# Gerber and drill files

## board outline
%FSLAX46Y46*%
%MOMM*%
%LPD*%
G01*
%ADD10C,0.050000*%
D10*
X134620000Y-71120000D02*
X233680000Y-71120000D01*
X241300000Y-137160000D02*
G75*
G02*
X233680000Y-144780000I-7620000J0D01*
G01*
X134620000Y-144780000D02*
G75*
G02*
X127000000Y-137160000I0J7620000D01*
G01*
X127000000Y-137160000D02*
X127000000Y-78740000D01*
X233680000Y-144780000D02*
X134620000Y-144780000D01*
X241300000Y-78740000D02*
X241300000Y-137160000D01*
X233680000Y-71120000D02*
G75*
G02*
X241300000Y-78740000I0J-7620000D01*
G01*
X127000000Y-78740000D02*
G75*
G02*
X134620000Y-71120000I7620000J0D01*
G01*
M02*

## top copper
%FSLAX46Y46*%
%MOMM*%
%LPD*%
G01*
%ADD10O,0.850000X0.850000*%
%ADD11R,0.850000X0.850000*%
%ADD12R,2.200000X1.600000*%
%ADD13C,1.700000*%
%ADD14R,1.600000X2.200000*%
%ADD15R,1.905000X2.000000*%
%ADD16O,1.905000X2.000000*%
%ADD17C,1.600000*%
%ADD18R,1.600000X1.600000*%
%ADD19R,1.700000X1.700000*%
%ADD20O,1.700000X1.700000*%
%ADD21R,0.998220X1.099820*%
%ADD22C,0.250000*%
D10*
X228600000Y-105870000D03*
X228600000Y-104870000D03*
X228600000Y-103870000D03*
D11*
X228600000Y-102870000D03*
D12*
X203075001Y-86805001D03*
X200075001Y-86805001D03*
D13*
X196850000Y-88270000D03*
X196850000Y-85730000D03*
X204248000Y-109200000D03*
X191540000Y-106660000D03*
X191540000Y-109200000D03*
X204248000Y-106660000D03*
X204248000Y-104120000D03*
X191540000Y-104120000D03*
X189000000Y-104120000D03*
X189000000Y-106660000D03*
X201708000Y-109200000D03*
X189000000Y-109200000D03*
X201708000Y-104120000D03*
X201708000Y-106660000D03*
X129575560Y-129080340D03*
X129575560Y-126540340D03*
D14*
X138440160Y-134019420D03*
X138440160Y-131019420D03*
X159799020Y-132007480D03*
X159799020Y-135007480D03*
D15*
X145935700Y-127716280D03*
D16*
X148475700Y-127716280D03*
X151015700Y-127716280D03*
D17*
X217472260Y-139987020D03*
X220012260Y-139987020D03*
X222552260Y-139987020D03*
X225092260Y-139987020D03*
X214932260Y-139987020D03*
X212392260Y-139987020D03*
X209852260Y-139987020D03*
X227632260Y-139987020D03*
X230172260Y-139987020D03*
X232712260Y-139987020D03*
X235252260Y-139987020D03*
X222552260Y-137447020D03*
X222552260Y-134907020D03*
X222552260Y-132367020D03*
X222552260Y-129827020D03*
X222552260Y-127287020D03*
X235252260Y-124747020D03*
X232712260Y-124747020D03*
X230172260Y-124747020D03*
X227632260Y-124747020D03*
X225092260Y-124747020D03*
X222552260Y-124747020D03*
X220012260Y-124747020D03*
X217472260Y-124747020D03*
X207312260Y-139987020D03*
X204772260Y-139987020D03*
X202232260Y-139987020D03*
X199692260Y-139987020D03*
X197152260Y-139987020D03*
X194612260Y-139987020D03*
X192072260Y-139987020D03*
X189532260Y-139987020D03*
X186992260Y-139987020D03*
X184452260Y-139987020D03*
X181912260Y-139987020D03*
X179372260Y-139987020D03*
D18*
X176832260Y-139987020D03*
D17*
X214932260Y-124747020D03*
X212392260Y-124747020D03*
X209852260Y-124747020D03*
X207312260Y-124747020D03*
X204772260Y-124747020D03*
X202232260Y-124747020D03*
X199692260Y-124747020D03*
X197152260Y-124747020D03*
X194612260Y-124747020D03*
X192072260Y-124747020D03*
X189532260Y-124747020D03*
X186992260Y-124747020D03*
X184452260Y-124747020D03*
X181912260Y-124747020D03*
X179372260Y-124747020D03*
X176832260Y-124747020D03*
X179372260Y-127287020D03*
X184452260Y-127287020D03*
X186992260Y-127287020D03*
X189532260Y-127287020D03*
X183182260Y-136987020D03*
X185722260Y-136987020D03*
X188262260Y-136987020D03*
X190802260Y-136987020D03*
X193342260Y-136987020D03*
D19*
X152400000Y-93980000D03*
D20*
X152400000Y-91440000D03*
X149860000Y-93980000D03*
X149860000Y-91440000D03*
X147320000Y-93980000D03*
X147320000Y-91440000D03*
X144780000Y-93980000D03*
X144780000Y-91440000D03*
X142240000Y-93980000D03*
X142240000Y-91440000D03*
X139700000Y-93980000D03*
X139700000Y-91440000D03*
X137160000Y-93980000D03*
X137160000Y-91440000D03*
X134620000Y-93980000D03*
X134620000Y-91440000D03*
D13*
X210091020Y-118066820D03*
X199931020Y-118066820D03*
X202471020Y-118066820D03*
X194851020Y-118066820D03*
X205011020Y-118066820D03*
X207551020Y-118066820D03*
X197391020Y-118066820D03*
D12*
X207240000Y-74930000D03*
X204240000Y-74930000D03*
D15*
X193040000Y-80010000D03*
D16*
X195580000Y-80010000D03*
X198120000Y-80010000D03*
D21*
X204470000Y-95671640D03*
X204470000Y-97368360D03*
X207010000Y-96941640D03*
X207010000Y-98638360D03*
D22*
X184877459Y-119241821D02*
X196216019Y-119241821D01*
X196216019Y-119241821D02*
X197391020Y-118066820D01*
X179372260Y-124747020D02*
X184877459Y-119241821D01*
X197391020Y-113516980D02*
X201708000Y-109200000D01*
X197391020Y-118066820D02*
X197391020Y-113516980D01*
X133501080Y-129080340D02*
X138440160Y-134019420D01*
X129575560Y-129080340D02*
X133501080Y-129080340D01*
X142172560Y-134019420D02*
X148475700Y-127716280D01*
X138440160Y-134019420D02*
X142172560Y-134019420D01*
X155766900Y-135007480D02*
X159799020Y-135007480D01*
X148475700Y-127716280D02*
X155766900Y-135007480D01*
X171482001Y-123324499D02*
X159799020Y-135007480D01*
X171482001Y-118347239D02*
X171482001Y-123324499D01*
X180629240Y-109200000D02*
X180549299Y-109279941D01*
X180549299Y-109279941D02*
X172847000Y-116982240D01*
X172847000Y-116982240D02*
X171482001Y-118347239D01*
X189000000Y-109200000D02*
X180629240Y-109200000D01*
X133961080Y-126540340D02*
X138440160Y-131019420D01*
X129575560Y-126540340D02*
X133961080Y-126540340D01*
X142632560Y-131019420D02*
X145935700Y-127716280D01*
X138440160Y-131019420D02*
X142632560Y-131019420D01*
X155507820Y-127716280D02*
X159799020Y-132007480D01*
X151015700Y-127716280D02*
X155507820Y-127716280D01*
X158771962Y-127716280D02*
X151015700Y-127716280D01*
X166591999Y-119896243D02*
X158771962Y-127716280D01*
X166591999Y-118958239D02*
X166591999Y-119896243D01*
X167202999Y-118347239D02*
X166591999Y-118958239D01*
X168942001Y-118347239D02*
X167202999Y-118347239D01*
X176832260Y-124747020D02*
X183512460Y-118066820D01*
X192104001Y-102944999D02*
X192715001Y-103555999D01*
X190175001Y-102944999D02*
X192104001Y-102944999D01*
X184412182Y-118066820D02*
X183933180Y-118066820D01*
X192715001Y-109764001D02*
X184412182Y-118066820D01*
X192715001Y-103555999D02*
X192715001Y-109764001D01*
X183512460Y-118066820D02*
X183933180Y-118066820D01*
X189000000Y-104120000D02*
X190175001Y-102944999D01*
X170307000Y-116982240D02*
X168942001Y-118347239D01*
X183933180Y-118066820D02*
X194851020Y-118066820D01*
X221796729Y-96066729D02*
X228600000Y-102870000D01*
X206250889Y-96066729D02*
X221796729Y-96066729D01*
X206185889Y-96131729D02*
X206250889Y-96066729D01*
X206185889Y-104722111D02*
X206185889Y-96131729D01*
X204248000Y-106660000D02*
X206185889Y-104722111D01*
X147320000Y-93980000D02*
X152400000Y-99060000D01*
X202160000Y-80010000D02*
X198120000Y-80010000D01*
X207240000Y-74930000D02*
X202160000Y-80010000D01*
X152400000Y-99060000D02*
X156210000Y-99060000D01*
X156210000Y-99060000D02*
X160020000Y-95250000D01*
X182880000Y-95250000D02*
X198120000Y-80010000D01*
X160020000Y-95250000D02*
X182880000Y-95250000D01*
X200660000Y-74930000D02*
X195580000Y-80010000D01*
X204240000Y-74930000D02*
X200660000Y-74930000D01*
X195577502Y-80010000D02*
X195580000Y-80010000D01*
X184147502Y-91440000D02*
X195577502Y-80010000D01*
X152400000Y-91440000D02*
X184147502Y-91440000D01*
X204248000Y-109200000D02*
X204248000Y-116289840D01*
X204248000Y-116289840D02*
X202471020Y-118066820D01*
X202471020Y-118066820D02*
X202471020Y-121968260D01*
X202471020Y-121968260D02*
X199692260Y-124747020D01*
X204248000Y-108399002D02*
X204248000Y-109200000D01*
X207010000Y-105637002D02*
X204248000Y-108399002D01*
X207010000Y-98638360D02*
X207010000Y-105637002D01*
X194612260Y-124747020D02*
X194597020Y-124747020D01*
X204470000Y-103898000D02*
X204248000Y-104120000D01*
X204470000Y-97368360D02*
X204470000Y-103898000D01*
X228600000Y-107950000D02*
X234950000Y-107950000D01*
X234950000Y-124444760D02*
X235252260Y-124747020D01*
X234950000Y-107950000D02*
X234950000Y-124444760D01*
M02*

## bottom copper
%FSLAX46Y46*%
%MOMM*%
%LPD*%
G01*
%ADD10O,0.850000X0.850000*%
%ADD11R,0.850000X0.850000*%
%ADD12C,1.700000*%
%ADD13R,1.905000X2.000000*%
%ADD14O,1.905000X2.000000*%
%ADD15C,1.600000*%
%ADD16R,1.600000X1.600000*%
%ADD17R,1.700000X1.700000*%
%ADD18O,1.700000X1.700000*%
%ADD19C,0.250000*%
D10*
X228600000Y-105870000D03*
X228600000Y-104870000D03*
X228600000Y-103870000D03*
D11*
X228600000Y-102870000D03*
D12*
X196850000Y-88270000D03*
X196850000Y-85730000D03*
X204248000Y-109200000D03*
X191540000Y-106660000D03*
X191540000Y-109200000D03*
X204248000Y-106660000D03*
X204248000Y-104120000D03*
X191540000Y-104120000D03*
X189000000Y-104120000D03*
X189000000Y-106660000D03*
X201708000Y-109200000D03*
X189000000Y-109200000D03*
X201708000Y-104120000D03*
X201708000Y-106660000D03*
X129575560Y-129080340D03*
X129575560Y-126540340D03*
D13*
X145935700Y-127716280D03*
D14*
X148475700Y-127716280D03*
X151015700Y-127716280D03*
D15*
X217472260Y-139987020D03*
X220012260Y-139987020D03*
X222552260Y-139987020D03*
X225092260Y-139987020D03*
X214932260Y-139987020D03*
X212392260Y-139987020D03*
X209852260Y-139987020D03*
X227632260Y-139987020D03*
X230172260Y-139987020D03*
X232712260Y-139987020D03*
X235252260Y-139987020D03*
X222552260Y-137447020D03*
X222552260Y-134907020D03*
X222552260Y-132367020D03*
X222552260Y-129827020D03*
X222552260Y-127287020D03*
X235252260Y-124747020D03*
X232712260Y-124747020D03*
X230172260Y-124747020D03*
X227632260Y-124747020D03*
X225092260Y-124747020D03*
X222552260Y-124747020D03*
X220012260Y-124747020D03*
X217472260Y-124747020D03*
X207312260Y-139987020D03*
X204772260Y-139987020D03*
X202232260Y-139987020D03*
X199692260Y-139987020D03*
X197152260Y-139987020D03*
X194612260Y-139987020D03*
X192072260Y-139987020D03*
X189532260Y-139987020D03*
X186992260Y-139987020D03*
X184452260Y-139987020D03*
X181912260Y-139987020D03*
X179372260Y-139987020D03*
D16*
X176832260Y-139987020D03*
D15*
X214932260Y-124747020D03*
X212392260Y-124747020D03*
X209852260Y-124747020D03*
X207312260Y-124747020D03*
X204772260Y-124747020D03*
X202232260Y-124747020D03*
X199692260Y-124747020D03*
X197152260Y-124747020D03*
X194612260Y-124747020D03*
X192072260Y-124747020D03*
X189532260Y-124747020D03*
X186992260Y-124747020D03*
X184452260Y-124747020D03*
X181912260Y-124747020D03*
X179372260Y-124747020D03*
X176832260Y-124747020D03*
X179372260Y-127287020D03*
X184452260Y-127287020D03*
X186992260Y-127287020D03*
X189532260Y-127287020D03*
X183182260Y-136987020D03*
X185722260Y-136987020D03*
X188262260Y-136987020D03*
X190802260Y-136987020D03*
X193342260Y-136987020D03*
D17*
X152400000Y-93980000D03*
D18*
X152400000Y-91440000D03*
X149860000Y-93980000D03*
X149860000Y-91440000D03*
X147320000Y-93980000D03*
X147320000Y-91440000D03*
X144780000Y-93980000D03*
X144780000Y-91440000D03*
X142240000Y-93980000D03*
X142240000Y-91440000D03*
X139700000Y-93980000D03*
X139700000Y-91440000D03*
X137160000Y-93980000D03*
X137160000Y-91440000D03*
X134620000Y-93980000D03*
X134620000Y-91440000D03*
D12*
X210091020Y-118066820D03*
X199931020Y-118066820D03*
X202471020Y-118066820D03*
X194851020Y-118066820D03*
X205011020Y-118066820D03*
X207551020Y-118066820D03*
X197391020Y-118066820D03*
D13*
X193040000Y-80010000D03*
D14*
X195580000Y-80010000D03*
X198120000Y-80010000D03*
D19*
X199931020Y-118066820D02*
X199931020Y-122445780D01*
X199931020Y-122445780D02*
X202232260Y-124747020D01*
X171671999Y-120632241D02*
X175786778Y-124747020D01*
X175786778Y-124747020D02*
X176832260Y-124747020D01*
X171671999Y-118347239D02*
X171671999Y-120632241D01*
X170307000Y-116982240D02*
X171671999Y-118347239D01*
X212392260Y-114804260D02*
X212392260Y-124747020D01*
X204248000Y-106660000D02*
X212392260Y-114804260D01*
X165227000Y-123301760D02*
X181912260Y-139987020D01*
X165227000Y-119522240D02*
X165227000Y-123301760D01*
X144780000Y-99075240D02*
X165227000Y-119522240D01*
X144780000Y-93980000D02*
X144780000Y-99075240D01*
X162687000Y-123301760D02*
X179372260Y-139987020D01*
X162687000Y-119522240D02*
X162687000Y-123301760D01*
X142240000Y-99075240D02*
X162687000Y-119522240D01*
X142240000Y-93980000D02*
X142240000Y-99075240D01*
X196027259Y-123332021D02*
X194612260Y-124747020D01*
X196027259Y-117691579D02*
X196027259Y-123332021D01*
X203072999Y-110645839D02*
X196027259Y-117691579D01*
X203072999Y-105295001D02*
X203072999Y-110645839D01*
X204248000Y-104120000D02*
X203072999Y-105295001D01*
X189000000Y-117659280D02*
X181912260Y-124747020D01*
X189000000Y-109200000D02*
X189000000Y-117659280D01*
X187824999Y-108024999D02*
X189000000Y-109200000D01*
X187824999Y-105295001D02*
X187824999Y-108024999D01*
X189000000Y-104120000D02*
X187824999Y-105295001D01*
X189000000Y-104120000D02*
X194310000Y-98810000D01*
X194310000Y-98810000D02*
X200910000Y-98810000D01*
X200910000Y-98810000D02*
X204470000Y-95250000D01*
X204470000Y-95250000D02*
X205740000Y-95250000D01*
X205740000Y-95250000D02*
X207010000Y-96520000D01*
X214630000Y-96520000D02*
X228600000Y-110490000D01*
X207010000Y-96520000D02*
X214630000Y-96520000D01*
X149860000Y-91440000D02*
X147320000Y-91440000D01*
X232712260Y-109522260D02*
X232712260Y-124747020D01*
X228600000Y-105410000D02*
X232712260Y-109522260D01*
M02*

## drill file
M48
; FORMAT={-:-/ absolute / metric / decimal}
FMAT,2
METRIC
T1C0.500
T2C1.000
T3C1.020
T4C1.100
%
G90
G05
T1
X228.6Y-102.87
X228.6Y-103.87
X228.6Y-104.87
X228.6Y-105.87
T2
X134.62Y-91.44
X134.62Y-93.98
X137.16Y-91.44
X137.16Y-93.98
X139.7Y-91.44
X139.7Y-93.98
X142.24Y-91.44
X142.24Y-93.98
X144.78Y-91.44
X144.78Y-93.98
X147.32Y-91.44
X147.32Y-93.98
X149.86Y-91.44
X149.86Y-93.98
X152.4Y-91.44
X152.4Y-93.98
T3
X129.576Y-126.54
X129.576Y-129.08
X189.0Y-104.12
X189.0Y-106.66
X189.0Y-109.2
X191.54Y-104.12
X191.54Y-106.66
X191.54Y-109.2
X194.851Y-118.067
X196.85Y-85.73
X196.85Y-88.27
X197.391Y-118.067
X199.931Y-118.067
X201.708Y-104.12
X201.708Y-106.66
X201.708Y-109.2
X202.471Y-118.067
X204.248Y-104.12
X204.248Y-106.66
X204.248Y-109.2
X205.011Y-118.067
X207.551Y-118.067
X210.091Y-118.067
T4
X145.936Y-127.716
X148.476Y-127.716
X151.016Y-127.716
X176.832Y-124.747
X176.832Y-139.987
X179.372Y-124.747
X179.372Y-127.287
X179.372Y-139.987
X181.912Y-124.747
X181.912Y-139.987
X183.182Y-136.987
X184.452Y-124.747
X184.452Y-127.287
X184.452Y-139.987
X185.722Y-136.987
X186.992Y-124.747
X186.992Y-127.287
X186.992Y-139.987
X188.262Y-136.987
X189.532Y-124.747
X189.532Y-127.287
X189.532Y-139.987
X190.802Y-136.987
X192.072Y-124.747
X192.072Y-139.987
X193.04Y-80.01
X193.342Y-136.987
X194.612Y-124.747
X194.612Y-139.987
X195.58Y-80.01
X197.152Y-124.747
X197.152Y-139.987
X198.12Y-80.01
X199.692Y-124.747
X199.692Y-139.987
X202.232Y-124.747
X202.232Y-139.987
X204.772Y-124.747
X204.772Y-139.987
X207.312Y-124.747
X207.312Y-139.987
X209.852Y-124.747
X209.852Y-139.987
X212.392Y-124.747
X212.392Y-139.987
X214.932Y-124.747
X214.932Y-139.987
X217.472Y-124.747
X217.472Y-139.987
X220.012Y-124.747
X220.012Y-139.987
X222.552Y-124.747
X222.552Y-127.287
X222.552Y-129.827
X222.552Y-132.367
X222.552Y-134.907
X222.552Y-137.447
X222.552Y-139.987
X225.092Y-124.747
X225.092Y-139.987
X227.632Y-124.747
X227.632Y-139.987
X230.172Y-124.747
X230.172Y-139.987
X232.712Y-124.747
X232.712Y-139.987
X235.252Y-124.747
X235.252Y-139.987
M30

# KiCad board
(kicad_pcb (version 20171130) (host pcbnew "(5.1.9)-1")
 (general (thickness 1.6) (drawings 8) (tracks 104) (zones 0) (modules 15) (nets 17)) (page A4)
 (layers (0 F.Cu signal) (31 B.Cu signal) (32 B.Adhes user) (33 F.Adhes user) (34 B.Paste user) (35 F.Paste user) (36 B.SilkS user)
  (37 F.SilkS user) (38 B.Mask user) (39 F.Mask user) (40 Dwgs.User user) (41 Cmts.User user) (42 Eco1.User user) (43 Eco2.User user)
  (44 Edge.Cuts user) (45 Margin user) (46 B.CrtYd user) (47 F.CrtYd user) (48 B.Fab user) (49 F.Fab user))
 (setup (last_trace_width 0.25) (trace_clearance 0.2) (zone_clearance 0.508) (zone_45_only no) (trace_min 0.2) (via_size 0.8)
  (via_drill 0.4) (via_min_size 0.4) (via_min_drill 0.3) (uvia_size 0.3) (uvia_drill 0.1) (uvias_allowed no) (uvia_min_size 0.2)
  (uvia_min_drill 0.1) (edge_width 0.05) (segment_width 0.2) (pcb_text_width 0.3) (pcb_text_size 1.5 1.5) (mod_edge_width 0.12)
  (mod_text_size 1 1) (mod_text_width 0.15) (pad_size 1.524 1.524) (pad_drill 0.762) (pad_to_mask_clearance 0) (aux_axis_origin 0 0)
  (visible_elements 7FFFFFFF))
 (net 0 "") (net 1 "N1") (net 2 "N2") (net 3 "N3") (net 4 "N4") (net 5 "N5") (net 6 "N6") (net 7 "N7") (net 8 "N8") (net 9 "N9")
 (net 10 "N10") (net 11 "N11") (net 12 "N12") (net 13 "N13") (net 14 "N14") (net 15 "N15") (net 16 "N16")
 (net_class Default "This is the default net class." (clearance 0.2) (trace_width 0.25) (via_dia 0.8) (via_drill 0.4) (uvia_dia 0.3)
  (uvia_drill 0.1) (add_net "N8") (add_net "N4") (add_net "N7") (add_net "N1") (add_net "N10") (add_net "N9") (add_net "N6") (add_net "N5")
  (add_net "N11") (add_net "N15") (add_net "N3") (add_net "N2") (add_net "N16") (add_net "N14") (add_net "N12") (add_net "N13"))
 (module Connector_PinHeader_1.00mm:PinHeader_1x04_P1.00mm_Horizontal (layer F.Cu) (at 228.6 102.87)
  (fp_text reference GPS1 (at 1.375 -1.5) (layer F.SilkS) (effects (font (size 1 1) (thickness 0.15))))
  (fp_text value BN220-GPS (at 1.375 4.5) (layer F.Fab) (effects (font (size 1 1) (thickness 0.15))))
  (pad 4 thru_hole oval (at 0 3) (size 0.85 0.85) (drill 0.5) (layers *.Cu *.Mask) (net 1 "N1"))
  (pad 3 thru_hole oval (at 0 2) (size 0.85 0.85) (drill 0.5) (layers *.Cu *.Mask) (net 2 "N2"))
  (pad 2 thru_hole oval (at 0 1) (size 0.85 0.85) (drill 0.5) (layers *.Cu *.Mask) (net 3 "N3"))
  (pad 1 thru_hole rect (at 0 0) (size 0.85 0.85) (drill 0.5) (layers *.Cu *.Mask) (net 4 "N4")))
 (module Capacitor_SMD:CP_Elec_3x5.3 (layer F.Cu) (at 201.575001 86.805001)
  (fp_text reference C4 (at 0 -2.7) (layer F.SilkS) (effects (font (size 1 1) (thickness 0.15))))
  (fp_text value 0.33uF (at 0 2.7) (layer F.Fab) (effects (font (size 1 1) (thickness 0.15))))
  (pad 2 smd rect (at 1.5 0) (size 2.2 1.6) (layers F.Cu F.Paste F.Mask) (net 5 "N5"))
  (pad 1 smd rect (at -1.5 0) (size 2.2 1.6) (layers F.Cu F.Paste F.Mask) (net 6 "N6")))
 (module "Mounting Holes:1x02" (layer F.Cu) (at 196.85 91.44)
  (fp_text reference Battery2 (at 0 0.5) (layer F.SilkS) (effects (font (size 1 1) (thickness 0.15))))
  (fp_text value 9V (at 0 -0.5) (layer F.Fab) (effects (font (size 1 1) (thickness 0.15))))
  (pad 1 thru_hole circle (at 0 -3.17) (size 1.7 1.7) (drill 1.02) (layers *.Cu *.Mask) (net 6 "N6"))
  (pad 2 thru_hole circle (at 0 -5.71) (size 1.7 1.7) (drill 1.02) (layers *.Cu *.Mask) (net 5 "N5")))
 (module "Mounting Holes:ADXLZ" (layer F.Cu) (at 189 109.2)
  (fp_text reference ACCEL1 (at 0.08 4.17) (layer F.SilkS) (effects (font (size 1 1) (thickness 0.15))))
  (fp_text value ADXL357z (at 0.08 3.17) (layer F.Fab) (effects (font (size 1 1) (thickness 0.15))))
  (pad 3 thru_hole circle (at 15.248 0) (size 1.7 1.7) (drill 1.02) (layers *.Cu *.Mask) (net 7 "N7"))
  (pad 13 thru_hole circle (at 2.54 -2.54) (size 1.7 1.7) (drill 1.02) (layers *.Cu *.Mask))
  (pad 14 thru_hole circle (at 2.54 0) (size 1.7 1.7) (drill 1.02) (layers *.Cu *.Mask))
  (pad 2 thru_hole circle (at 15.248 -2.54) (size 1.7 1.7) (drill 1.02) (layers *.Cu *.Mask) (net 4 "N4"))
  (pad 1 thru_hole circle (at 15.248 -5.08) (size 1.7 1.7) (drill 1.02) (layers *.Cu *.Mask) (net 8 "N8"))
  (pad 12 thru_hole circle (at 2.54 -5.08) (size 1.7 1.7) (drill 1.02) (layers *.Cu *.Mask))
  (pad 5 thru_hole circle (at 0 -5.08) (size 1.7 1.7) (drill 1.02) (layers *.Cu *.Mask) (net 1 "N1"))
  (pad 11 thru_hole circle (at 0 -2.54) (size 1.7 1.7) (drill 1.02) (layers *.Cu *.Mask))
  (pad 4 thru_hole circle (at 12.708 0) (size 1.7 1.7) (drill 1.02) (layers *.Cu *.Mask))
  (pad 6 thru_hole circle (at 0 0) (size 1.7 1.7) (drill 1.02) (layers *.Cu *.Mask) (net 1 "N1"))
  (pad 10 thru_hole circle (at 12.708 -5.08) (size 1.7 1.7) (drill 1.02) (layers *.Cu *.Mask))
  (pad 8 thru_hole circle (at 12.708 -2.54) (size 1.7 1.7) (drill 1.02) (layers *.Cu *.Mask)))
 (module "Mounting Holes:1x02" (layer F.Cu) (at 129.57556 123.37034 180)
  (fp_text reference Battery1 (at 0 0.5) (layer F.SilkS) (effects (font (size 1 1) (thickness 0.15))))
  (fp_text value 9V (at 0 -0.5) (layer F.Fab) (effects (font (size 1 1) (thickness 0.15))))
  (pad 2 thru_hole circle (at 0 -5.71 180) (size 1.7 1.7) (drill 1.02) (layers *.Cu *.Mask) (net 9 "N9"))
  (pad 1 thru_hole circle (at 0 -3.17 180) (size 1.7 1.7) (drill 1.02) (layers *.Cu *.Mask) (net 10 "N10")))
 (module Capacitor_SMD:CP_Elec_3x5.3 (layer F.Cu) (at 138.44016 132.51942 270)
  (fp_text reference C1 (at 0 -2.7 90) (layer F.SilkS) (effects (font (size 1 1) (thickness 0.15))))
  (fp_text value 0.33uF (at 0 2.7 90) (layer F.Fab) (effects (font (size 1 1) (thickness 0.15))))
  (pad 2 smd rect (at 1.5 0 270) (size 2.2 1.6) (layers F.Cu F.Paste F.Mask) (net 9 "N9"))
  (pad 1 smd rect (at -1.5 0 270) (size 2.2 1.6) (layers F.Cu F.Paste F.Mask) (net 10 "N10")))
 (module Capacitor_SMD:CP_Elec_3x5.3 (layer F.Cu) (at 159.79902 133.50748 270)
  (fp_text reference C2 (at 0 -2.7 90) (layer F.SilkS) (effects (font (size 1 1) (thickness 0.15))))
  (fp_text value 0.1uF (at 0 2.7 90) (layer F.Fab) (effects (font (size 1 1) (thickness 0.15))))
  (pad 1 smd rect (at -1.5 0 270) (size 2.2 1.6) (layers F.Cu F.Paste F.Mask) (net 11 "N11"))
  (pad 2 smd rect (at 1.5 0 270) (size 2.2 1.6) (layers F.Cu F.Paste F.Mask) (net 9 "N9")))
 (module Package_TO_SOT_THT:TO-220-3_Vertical (layer F.Cu) (at 145.9357 127.71628)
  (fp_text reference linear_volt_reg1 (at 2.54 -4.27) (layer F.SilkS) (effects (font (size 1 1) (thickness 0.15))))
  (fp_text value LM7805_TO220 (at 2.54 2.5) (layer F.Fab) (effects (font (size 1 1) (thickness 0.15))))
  (pad 1 thru_hole rect (at 0 0) (size 1.905 2) (drill 1.1) (layers *.Cu *.Mask) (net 10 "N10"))
  (pad 2 thru_hole oval (at 2.54 0) (size 1.905 2) (drill 1.1) (layers *.Cu *.Mask) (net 9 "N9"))
  (pad 3 thru_hole oval (at 5.08 0) (size 1.905 2) (drill 1.1) (layers *.Cu *.Mask) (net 11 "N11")))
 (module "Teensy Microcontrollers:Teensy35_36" (layer F.Cu) (at 206.04226 132.36702)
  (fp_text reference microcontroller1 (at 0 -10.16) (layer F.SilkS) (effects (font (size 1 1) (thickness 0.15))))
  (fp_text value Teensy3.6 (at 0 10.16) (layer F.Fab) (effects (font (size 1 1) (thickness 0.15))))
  (pad 17 thru_hole circle (at 11.43 7.62) (size 1.6 1.6) (drill 1.1) (layers *.Cu *.Mask))
  (pad 18 thru_hole circle (at 13.97 7.62) (size 1.6 1.6) (drill 1.1) (layers *.Cu *.Mask))
  (pad 19 thru_hole circle (at 16.51 7.62) (size 1.6 1.6) (drill 1.1) (layers *.Cu *.Mask))
  (pad 20 thru_hole circle (at 19.05 7.62) (size 1.6 1.6) (drill 1.1) (layers *.Cu *.Mask))
  (pad 16 thru_hole circle (at 8.89 7.62) (size 1.6 1.6) (drill 1.1) (layers *.Cu *.Mask))
  (pad 15 thru_hole circle (at 6.35 7.62) (size 1.6 1.6) (drill 1.1) (layers *.Cu *.Mask))
  (pad 14 thru_hole circle (at 3.81 7.62) (size 1.6 1.6) (drill 1.1) (layers *.Cu *.Mask))
  (pad 21 thru_hole circle (at 21.59 7.62) (size 1.6 1.6) (drill 1.1) (layers *.Cu *.Mask))
  (pad 22 thru_hole circle (at 24.13 7.62) (size 1.6 1.6) (drill 1.1) (layers *.Cu *.Mask))
  (pad 23 thru_hole circle (at 26.67 7.62) (size 1.6 1.6) (drill 1.1) (layers *.Cu *.Mask))
  (pad 24 thru_hole circle (at 29.21 7.62) (size 1.6 1.6) (drill 1.1) (layers *.Cu *.Mask))
  (pad 25 thru_hole circle (at 16.51 5.08) (size 1.6 1.6) (drill 1.1) (layers *.Cu *.Mask))
  (pad 26 thru_hole circle (at 16.51 2.54) (size 1.6 1.6) (drill 1.1) (layers *.Cu *.Mask))
  (pad 27 thru_hole circle (at 16.51 0) (size 1.6 1.6) (drill 1.1) (layers *.Cu *.Mask))
  (pad 28 thru_hole circle (at 16.51 -2.54) (size 1.6 1.6) (drill 1.1) (layers *.Cu *.Mask))
  (pad 29 thru_hole circle (at 16.51 -5.08) (size 1.6 1.6) (drill 1.1) (layers *.Cu *.Mask))
  (pad 30 thru_hole circle (at 29.21 -7.62) (size 1.6 1.6) (drill 1.1) (layers *.Cu *.Mask) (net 2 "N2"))
  (pad 31 thru_hole circle (at 26.67 -7.62) (size 1.6 1.6) (drill 1.1) (layers *.Cu *.Mask) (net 3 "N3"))
  (pad 32 thru_hole circle (at 24.13 -7.62) (size 1.6 1.6) (drill 1.1) (layers *.Cu *.Mask))
  (pad 33 thru_hole circle (at 21.59 -7.62) (size 1.6 1.6) (drill 1.1) (layers *.Cu *.Mask))
  (pad 34 thru_hole circle (at 19.05 -7.62) (size 1.6 1.6) (drill 1.1) (layers *.Cu *.Mask))
  (pad 35 thru_hole circle (at 16.51 -7.62) (size 1.6 1.6) (drill 1.1) (layers *.Cu *.Mask))
  (pad 36 thru_hole circle (at 13.97 -7.62) (size 1.6 1.6) (drill 1.1) (layers *.Cu *.Mask))
  (pad 37 thru_hole circle (at 11.43 -7.62) (size 1.6 1.6) (drill 1.1) (layers *.Cu *.Mask))
  (pad 13 thru_hole circle (at 1.27 7.62) (size 1.6 1.6) (drill 1.1) (layers *.Cu *.Mask))
  (pad 12 thru_hole circle (at -1.27 7.62) (size 1.6 1.6) (drill 1.1) (layers *.Cu *.Mask))
  (pad 11 thru_hole circle (at -3.81 7.62) (size 1.6 1.6) (drill 1.1) (layers *.Cu *.Mask))
  (pad 10 thru_hole circle (at -6.35 7.62) (size 1.6 1.6) (drill 1.1) (layers *.Cu *.Mask))
  (pad 9 thru_hole circle (at -8.89 7.62) (size 1.6 1.6) (drill 1.1) (layers *.Cu *.Mask))
  (pad 8 thru_hole circle (at -11.43 7.62) (size 1.6 1.6) (drill 1.1) (layers *.Cu *.Mask))
  (pad 7 thru_hole circle (at -13.97 7.62) (size 1.6 1.6) (drill 1.1) (layers *.Cu *.Mask))
  (pad 6 thru_hole circle (at -16.51 7.62) (size 1.6 1.6) (drill 1.1) (layers *.Cu *.Mask))
  (pad 5 thru_hole circle (at -19.05 7.62) (size 1.6 1.6) (drill 1.1) (layers *.Cu *.Mask))
  (pad 4 thru_hole circle (at -21.59 7.62) (size 1.6 1.6) (drill 1.1) (layers *.Cu *.Mask))
  (pad 3 thru_hole circle (at -24.13 7.62) (size 1.6 1.6) (drill 1.1) (layers *.Cu *.Mask) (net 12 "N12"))
  (pad 2 thru_hole circle (at -26.67 7.62) (size 1.6 1.6) (drill 1.1) (layers *.Cu *.Mask) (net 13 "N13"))
  (pad 1 thru_hole rect (at -29.21 7.62) (size 1.6 1.6) (drill 1.1) (layers *.Cu *.Mask))
  (pad 38 thru_hole circle (at 8.89 -7.62) (size 1.6 1.6) (drill 1.1) (layers *.Cu *.Mask))
  (pad 39 thru_hole circle (at 6.35 -7.62) (size 1.6 1.6) (drill 1.1) (layers *.Cu *.Mask) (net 4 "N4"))
  (pad 40 thru_hole circle (at 3.81 -7.62) (size 1.6 1.6) (drill 1.1) (layers *.Cu *.Mask))
  (pad 41 thru_hole circle (at 1.27 -7.62) (size 1.6 1.6) (drill 1.1) (layers *.Cu *.Mask))
  (pad 42 thru_hole circle (at -1.27 -7.62) (size 1.6 1.6) (drill 1.1) (layers *.Cu *.Mask))
  (pad 43 thru_hole circle (at -3.81 -7.62) (size 1.6 1.6) (drill 1.1) (layers *.Cu *.Mask))
  (pad 44 thru_hole circle (at -6.35 -7.62) (size 1.6 1.6) (drill 1.1) (layers *.Cu *.Mask))
  (pad 45 thru_hole circle (at -8.89 -7.62) (size 1.6 1.6) (drill 1.1) (layers *.Cu *.Mask) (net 7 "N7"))
  (pad 46 thru_hole circle (at -11.43 -7.62) (size 1.6 1.6) (drill 1.1) (layers *.Cu *.Mask) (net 8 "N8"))
  (pad 47 thru_hole circle (at -13.97 -7.62) (size 1.6 1.6) (drill 1.1) (layers *.Cu *.Mask))
  (pad 48 thru_hole circle (at -16.51 -7.62) (size 1.6 1.6) (drill 1.1) (layers *.Cu *.Mask))
  (pad 49 thru_hole circle (at -19.05 -7.62) (size 1.6 1.6) (drill 1.1) (layers *.Cu *.Mask))
  (pad 50 thru_hole circle (at -21.59 -7.62) (size 1.6 1.6) (drill 1.1) (layers *.Cu *.Mask))
  (pad 51 thru_hole circle (at -24.13 -7.62) (size 1.6 1.6) (drill 1.1) (layers *.Cu *.Mask) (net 1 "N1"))
  (pad 52 thru_hole circle (at -26.67 -7.62) (size 1.6 1.6) (drill 1.1) (layers *.Cu *.Mask))
  (pad 53 thru_hole circle (at -29.21 -7.62) (size 1.6 1.6) (drill 1.1) (layers *.Cu *.Mask) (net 11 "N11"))
  (pad 54 thru_hole circle (at -26.67 -5.08) (size 1.6 1.6) (drill 1.1) (layers *.Cu *.Mask))
  (pad 55 thru_hole circle (at -21.59 -5.08) (size 1.6 1.6) (drill 1.1) (layers *.Cu *.Mask))
  (pad 56 thru_hole circle (at -19.05 -5.08) (size 1.6 1.6) (drill 1.1) (layers *.Cu *.Mask))
  (pad 57 thru_hole circle (at -16.51 -5.08) (size 1.6 1.6) (drill 1.1) (layers *.Cu *.Mask))
  (pad 58 thru_hole circle (at -22.86 4.62) (size 1.6 1.6) (drill 1.1) (layers *.Cu *.Mask))
  (pad 59 thru_hole circle (at -20.32 4.62) (size 1.6 1.6) (drill 1.1) (layers *.Cu *.Mask))
  (pad 60 thru_hole circle (at -17.78 4.62) (size 1.6 1.6) (drill 1.1) (layers *.Cu *.Mask))
  (pad 61 thru_hole circle (at -15.24 4.62) (size 1.6 1.6) (drill 1.1) (layers *.Cu *.Mask))
  (pad 62 thru_hole circle (at -12.7 4.62) (size 1.6 1.6) (drill 1.1) (layers *.Cu *.Mask)))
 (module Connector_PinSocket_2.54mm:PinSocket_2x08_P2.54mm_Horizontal (layer F.Cu) (at 152.4 93.98 270)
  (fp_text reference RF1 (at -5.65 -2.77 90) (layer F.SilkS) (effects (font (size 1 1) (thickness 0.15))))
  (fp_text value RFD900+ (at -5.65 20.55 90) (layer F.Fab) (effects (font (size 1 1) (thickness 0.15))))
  (pad 1 thru_hole rect (at 0 0 270) (size 1.7 1.7) (drill 1) (layers *.Cu *.Mask))
  (pad 2 thru_hole oval (at -2.54 0 270) (size 1.7 1.7) (drill 1) (layers *.Cu *.Mask) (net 5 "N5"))
  (pad 3 thru_hole oval (at 0 2.54 270) (size 1.7 1.7) (drill 1) (layers *.Cu *.Mask))
  (pad 4 thru_hole oval (at -2.54 2.54 270) (size 1.7 1.7) (drill 1) (layers *.Cu *.Mask) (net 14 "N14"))
  (pad 5 thru_hole oval (at 0 5.08 270) (size 1.7 1.7) (drill 1) (layers *.Cu *.Mask) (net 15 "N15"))
  (pad 6 thru_hole oval (at -2.54 5.08 270) (size 1.7 1.7) (drill 1) (layers *.Cu *.Mask) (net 14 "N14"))
  (pad 7 thru_hole oval (at 0 7.62 270) (size 1.7 1.7) (drill 1) (layers *.Cu *.Mask) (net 12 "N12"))
  (pad 8 thru_hole oval (at -2.54 7.62 270) (size 1.7 1.7) (drill 1) (layers *.Cu *.Mask))
  (pad 9 thru_hole oval (at 0 10.16 270) (size 1.7 1.7) (drill 1) (layers *.Cu *.Mask) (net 13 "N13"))
  (pad 10 thru_hole oval (at -2.54 10.16 270) (size 1.7 1.7) (drill 1) (layers *.Cu *.Mask))
  (pad 11 thru_hole oval (at 0 12.7 270) (size 1.7 1.7) (drill 1) (layers *.Cu *.Mask))
  (pad 12 thru_hole oval (at -2.54 12.7 270) (size 1.7 1.7) (drill 1) (layers *.Cu *.Mask))
  (pad 13 thru_hole oval (at 0 15.24 270) (size 1.7 1.7) (drill 1) (layers *.Cu *.Mask))
  (pad 14 thru_hole oval (at -2.54 15.24 270) (size 1.7 1.7) (drill 1) (layers *.Cu *.Mask))
  (pad 15 thru_hole oval (at 0 17.78 270) (size 1.7 1.7) (drill 1) (layers *.Cu *.Mask))
  (pad 16 thru_hole oval (at -2.54 17.78 270) (size 1.7 1.7) (drill 1) (layers *.Cu *.Mask)))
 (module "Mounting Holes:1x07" (layer F.Cu) (at 192.53102 118.08682 270)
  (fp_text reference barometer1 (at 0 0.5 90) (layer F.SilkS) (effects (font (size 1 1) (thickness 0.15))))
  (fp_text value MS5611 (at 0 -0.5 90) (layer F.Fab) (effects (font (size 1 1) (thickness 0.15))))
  (pad 7 thru_hole circle (at -0.02 -17.56 270) (size 1.7 1.7) (drill 1.02) (layers *.Cu *.Mask))
  (pad 3 thru_hole circle (at -0.02 -7.4 270) (size 1.7 1.7) (drill 1.02) (layers *.Cu *.Mask))
  (pad 4 thru_hole circle (at -0.02 -9.94 270) (size 1.7 1.7) (drill 1.02) (layers *.Cu *.Mask))
  (pad 1 thru_hole circle (at -0.02 -2.32 270) (size 1.7 1.7) (drill 1.02) (layers *.Cu *.Mask))
  (pad 5 thru_hole circle (at -0.02 -12.48 270) (size 1.7 1.7) (drill 1.02) (layers *.Cu *.Mask))
  (pad 6 thru_hole circle (at -0.02 -15.02 270) (size 1.7 1.7) (drill 1.02) (layers *.Cu *.Mask))
  (pad 2 thru_hole circle (at -0.02 -4.86 270) (size 1.7 1.7) (drill 1.02) (layers *.Cu *.Mask)))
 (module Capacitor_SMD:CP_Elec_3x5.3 (layer F.Cu) (at 205.74 74.93 180)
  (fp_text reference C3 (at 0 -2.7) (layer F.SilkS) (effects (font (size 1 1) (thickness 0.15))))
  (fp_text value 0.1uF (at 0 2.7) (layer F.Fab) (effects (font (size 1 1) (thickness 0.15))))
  (pad 1 smd rect (at -1.5 0 180) (size 2.2 1.6) (layers F.Cu F.Paste F.Mask) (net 15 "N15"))
  (pad 2 smd rect (at 1.5 0 180) (size 2.2 1.6) (layers F.Cu F.Paste F.Mask) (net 5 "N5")))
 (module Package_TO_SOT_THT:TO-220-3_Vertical (layer F.Cu) (at 193.04 80.01)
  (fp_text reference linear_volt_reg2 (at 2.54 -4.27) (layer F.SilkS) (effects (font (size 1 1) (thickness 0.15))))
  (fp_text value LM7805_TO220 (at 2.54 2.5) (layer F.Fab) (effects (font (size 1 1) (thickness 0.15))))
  (pad 1 thru_hole rect (at 0 0) (size 1.905 2) (drill 1.1) (layers *.Cu *.Mask) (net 6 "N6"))
  (pad 2 thru_hole oval (at 2.54 0) (size 1.905 2) (drill 1.1) (layers *.Cu *.Mask) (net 5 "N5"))
  (pad 3 thru_hole oval (at 5.08 0) (size 1.905 2) (drill 1.1) (layers *.Cu *.Mask) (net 15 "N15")))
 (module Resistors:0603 (layer F.Cu) (at 204.47 96.52 270)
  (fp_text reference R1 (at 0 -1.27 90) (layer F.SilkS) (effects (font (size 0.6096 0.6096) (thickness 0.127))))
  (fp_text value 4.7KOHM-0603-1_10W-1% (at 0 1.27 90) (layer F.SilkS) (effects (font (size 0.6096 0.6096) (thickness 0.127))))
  (pad 1 smd rect (at -0.84836 0 270) (size 1.09982 0.99822) (layers F.Cu F.Paste F.Mask) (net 1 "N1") (solder_mask_margin 0.1016))
  (pad 2 smd rect (at 0.84836 0 270) (size 1.09982 0.99822) (layers F.Cu F.Paste F.Mask) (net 8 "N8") (solder_mask_margin 0.1016)))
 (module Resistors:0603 (layer F.Cu) (at 207.01 97.79 90)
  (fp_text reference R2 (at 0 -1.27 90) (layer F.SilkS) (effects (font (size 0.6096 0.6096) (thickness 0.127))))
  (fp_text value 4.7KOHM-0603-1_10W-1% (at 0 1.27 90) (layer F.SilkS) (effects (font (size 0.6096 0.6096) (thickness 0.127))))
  (pad 2 smd rect (at 0.84836 0 90) (size 1.09982 0.99822) (layers F.Cu F.Paste F.Mask) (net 1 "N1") (solder_mask_margin 0.1016))
  (pad 1 smd rect (at -0.84836 0 90) (size 1.09982 0.99822) (layers F.Cu F.Paste F.Mask) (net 7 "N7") (solder_mask_margin 0.1016)))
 (gr_line (start 134.62 71.12) (end 233.68 71.12) (layer Edge.Cuts) (width 0.05))
 (gr_arc (start 233.68 137.16) (end 233.68 144.78) (angle -90) (layer Edge.Cuts) (width 0.05))
 (gr_arc (start 134.62 137.16) (end 127 137.16) (angle -90) (layer Edge.Cuts) (width 0.05))
 (gr_line (start 127 137.16) (end 127 78.74) (layer Edge.Cuts) (width 0.05))
 (gr_line (start 233.68 144.78) (end 134.62 144.78) (layer Edge.Cuts) (width 0.05))
 (gr_line (start 241.3 78.74) (end 241.3 137.16) (layer Edge.Cuts) (width 0.05))
 (gr_arc (start 233.68 78.74) (end 241.3 78.74) (angle -90) (layer Edge.Cuts) (width 0.05))
 (gr_arc (start 134.62 78.74) (end 134.62 71.12) (angle -90) (layer Edge.Cuts) (width 0.05))
 (segment (start 184.877459 119.241821) (end 196.216019 119.241821) (width 0.25) (layer F.Cu) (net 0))
 (segment (start 196.216019 119.241821) (end 197.39102 118.06682) (width 0.25) (layer F.Cu) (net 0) (status 20))
 (segment (start 179.37226 124.74702) (end 184.877459 119.241821) (width 0.25) (layer F.Cu) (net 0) (status 10))
 (segment (start 197.39102 113.51698) (end 201.708 109.2) (width 0.25) (layer F.Cu) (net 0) (status 20))
 (segment (start 197.39102 118.06682) (end 197.39102 113.51698) (width 0.25) (layer F.Cu) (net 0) (status 10))
 (segment (start 199.93102 118.06682) (end 199.93102 122.44578) (width 0.25) (layer B.Cu) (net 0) (status 10))
 (segment (start 199.93102 122.44578) (end 202.23226 124.74702) (width 0.25) (layer B.Cu) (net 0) (status 20))
 (segment (start 133.50108 129.08034) (end 138.44016 134.01942) (width 0.25) (layer F.Cu) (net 9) (status 20))
 (segment (start 129.57556 129.08034) (end 133.50108 129.08034) (width 0.25) (layer F.Cu) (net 9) (status 10))
 (segment (start 142.17256 134.01942) (end 148.4757 127.71628) (width 0.25) (layer F.Cu) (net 9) (status 20))
 (segment (start 138.44016 134.01942) (end 142.17256 134.01942) (width 0.25) (layer F.Cu) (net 9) (status 10))
 (segment (start 155.7669 135.00748) (end 159.79902 135.00748) (width 0.25) (layer F.Cu) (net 9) (status 20))
 (segment (start 148.4757 127.71628) (end 155.7669 135.00748) (width 0.25) (layer F.Cu) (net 9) (status 10))
 (segment (start 171.482001 123.324499) (end 159.79902 135.00748) (width 0.25) (layer F.Cu) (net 9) (status 20))
 (segment (start 171.482001 118.347239) (end 171.482001 123.324499) (width 0.25) (layer F.Cu) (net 9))
 (segment (start 180.62924 109.2) (end 180.549299 109.279941) (width 0.25) (layer F.Cu) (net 9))
 (segment (start 180.549299 109.279941) (end 172.847 116.98224) (width 0.25) (layer F.Cu) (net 9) (status 20))
 (segment (start 172.847 116.98224) (end 171.482001 118.347239) (width 0.25) (layer F.Cu) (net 9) (status 10))
 (segment (start 189 109.2) (end 180.62924 109.2) (width 0.25) (layer F.Cu) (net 9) (status 10))
 (segment (start 133.96108 126.54034) (end 138.44016 131.01942) (width 0.25) (layer F.Cu) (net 10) (status 20))
 (segment (start 129.57556 126.54034) (end 133.96108 126.54034) (width 0.25) (layer F.Cu) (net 10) (status 10))
 (segment (start 142.63256 131.01942) (end 145.9357 127.71628) (width 0.25) (layer F.Cu) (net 10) (status 20))
 (segment (start 138.44016 131.01942) (end 142.63256 131.01942) (width 0.25) (layer F.Cu) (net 10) (status 10))
 (segment (start 155.50782 127.71628) (end 159.79902 132.00748) (width 0.25) (layer F.Cu) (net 11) (status 20))
 (segment (start 151.0157 127.71628) (end 155.50782 127.71628) (width 0.25) (layer F.Cu) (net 11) (status 10))
 (segment (start 158.771962 127.71628) (end 151.0157 127.71628) (width 0.25) (layer F.Cu) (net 11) (status 20))
 (segment (start 166.591999 119.896243) (end 158.771962 127.71628) (width 0.25) (layer F.Cu) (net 11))
 (segment (start 166.591999 118.958239) (end 166.591999 119.896243) (width 0.25) (layer F.Cu) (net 11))
 (segment (start 167.202999 118.347239) (end 166.591999 118.958239) (width 0.25) (layer F.Cu) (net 11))
 (segment (start 168.942001 118.347239) (end 167.202999 118.347239) (width 0.25) (layer F.Cu) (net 11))
 (segment (start 171.671999 120.632241) (end 175.786778 124.74702) (width 0.25) (layer B.Cu) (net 11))
 (segment (start 175.786778 124.74702) (end 176.83226 124.74702) (width 0.25) (layer B.Cu) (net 11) (status 20))
 (segment (start 171.671999 118.347239) (end 171.671999 120.632241) (width 0.25) (layer B.Cu) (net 11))
 (segment (start 176.83226 124.74702) (end 183.51246 118.06682) (width 0.25) (layer F.Cu) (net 11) (status 10))
 (segment (start 192.104001 102.944999) (end 192.715001 103.555999) (width 0.25) (layer F.Cu) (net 11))
 (segment (start 190.175001 102.944999) (end 192.104001 102.944999) (width 0.25) (layer F.Cu) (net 11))
 (segment (start 184.412182 118.06682) (end 183.93318 118.06682) (width 0.25) (layer F.Cu) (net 11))
 (segment (start 192.715001 109.764001) (end 184.412182 118.06682) (width 0.25) (layer F.Cu) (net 11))
 (segment (start 192.715001 103.555999) (end 192.715001 109.764001) (width 0.25) (layer F.Cu) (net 11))
 (segment (start 183.51246 118.06682) (end 183.93318 118.06682) (width 0.25) (layer F.Cu) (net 11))
 (segment (start 189 104.12) (end 190.175001 102.944999) (width 0.25) (layer F.Cu) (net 11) (status 10))
 (segment (start 170.307 116.98224) (end 168.942001 118.347239) (width 0.25) (layer F.Cu) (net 11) (status 10))
 (segment (start 183.93318 118.06682) (end 194.85102 118.06682) (width 0.25) (layer F.Cu) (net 11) (status 20))
 (segment (start 170.307 116.98224) (end 171.671999 118.347239) (width 0.25) (layer B.Cu) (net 11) (status 10))
 (segment (start 221.796729 96.066729) (end 228.6 102.87) (width 0.25) (layer F.Cu) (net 4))
 (segment (start 206.250889 96.066729) (end 221.796729 96.066729) (width 0.25) (layer F.Cu) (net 4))
 (segment (start 206.185889 96.131729) (end 206.250889 96.066729) (width 0.25) (layer F.Cu) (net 4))
 (segment (start 206.185889 104.722111) (end 206.185889 96.131729) (width 0.25) (layer F.Cu) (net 4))
 (segment (start 204.248 106.66) (end 206.185889 104.722111) (width 0.25) (layer F.Cu) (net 4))
 (segment (start 212.39226 114.80426) (end 212.39226 124.74702) (width 0.25) (layer B.Cu) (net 4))
 (segment (start 204.248 106.66) (end 212.39226 114.80426) (width 0.25) (layer B.Cu) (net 4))
 (segment (start 165.227 123.30176) (end 181.91226 139.98702) (width 0.25) (layer B.Cu) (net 12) (status 20))
 (segment (start 165.227 119.52224) (end 165.227 123.30176) (width 0.25) (layer B.Cu) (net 12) (status 10))
 (segment (start 144.78 99.07524) (end 165.227 119.52224) (width 0.25) (layer B.Cu) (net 12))
 (segment (start 144.78 93.98) (end 144.78 99.07524) (width 0.25) (layer B.Cu) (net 12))
 (segment (start 162.687 123.30176) (end 179.37226 139.98702) (width 0.25) (layer B.Cu) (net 13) (status 20))
 (segment (start 162.687 119.52224) (end 162.687 123.30176) (width 0.25) (layer B.Cu) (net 13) (status 10))
 (segment (start 142.24 99.07524) (end 162.687 119.52224) (width 0.25) (layer B.Cu) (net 13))
 (segment (start 142.24 93.98) (end 142.24 99.07524) (width 0.25) (layer B.Cu) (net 13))
 (segment (start 147.32 93.98) (end 152.4 99.06) (width 0.25) (layer F.Cu) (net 15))
 (segment (start 202.16 80.01) (end 198.12 80.01) (width 0.25) (layer F.Cu) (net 15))
 (segment (start 207.24 74.93) (end 202.16 80.01) (width 0.25) (layer F.Cu) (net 15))
 (segment (start 152.4 99.06) (end 156.21 99.06) (width 0.25) (layer F.Cu) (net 15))
 (segment (start 156.21 99.06) (end 160.02 95.25) (width 0.25) (layer F.Cu) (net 15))
 (segment (start 182.88 95.25) (end 198.12 80.01) (width 0.25) (layer F.Cu) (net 15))
 (segment (start 160.02 95.25) (end 182.88 95.25) (width 0.25) (layer F.Cu) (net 15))
 (segment (start 200.66 74.93) (end 195.58 80.01) (width 0.25) (layer F.Cu) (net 5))
 (segment (start 204.24 74.93) (end 200.66 74.93) (width 0.25) (layer F.Cu) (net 5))
 (segment (start 195.577502 80.01) (end 195.58 80.01) (width 0.25) (layer F.Cu) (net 5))
 (segment (start 184.147502 91.44) (end 195.577502 80.01) (width 0.25) (layer F.Cu) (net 5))
 (segment (start 152.4 91.44) (end 184.147502 91.44) (width 0.25) (layer F.Cu) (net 5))
 (segment (start 204.248 109.2) (end 204.248 116.28984) (width 0.25) (layer F.Cu) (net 7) (status 10))
 (segment (start 204.248 116.28984) (end 202.47102 118.06682) (width 0.25) (layer F.Cu) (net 7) (status 20))
 (segment (start 202.47102 118.06682) (end 202.47102 121.96826) (width 0.25) (layer F.Cu) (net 7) (status 10))
 (segment (start 202.47102 121.96826) (end 199.69226 124.74702) (width 0.25) (layer F.Cu) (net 7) (status 20))
 (segment (start 204.248 108.399002) (end 204.248 109.2) (width 0.25) (layer F.Cu) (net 7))
 (segment (start 207.01 105.637002) (end 204.248 108.399002) (width 0.25) (layer F.Cu) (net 7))
 (segment (start 207.01 98.63836) (end 207.01 105.637002) (width 0.25) (layer F.Cu) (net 7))
 (segment (start 194.61226 124.74702) (end 194.59702 124.74702) (width 0.25) (layer F.Cu) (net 8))
 (segment (start 204.47 103.898) (end 204.248 104.12) (width 0.25) (layer F.Cu) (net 8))
 (segment (start 204.47 97.36836) (end 204.47 103.898) (width 0.25) (layer F.Cu) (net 8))
 (segment (start 196.027259 123.332021) (end 194.61226 124.74702) (width 0.25) (layer B.Cu) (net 8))
 (segment (start 196.027259 117.691579) (end 196.027259 123.332021) (width 0.25) (layer B.Cu) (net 8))
 (segment (start 203.072999 110.645839) (end 196.027259 117.691579) (width 0.25) (layer B.Cu) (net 8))
 (segment (start 203.072999 105.295001) (end 203.072999 110.645839) (width 0.25) (layer B.Cu) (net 8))
 (segment (start 204.248 104.12) (end 203.072999 105.295001) (width 0.25) (layer B.Cu) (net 8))
 (segment (start 189 117.65928) (end 181.91226 124.74702) (width 0.25) (layer B.Cu) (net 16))
 (segment (start 189 109.2) (end 189 117.65928) (width 0.25) (layer B.Cu) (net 16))
 (segment (start 187.824999 108.024999) (end 189 109.2) (width 0.25) (layer B.Cu) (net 16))
 (segment (start 187.824999 105.295001) (end 187.824999 108.024999) (width 0.25) (layer B.Cu) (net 16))
 (segment (start 189 104.12) (end 187.824999 105.295001) (width 0.25) (layer B.Cu) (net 16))
 (segment (start 189 104.12) (end 194.31 98.81) (width 0.25) (layer B.Cu) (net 16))
 (segment (start 194.31 98.81) (end 200.91 98.81) (width 0.25) (layer B.Cu) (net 16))
 (segment (start 200.91 98.81) (end 204.47 95.25) (width 0.25) (layer B.Cu) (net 16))
 (segment (start 204.47 95.25) (end 205.74 95.25) (width 0.25) (layer B.Cu) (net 16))
 (segment (start 205.74 95.25) (end 207.01 96.52) (width 0.25) (layer B.Cu) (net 16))
 (segment (start 214.63 96.52) (end 228.6 110.49) (width 0.25) (layer B.Cu) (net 16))
 (segment (start 207.01 96.52) (end 214.63 96.52) (width 0.25) (layer B.Cu) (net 16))
 (segment (start 149.86 91.44) (end 147.32 91.44) (width 0.25) (layer B.Cu) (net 14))
 (segment (start 228.6 107.95) (end 234.95 107.95) (width 0.25) (layer F.Cu) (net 2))
 (segment (start 234.95 124.44476) (end 235.25226 124.74702) (width 0.25) (layer F.Cu) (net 2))
 (segment (start 234.95 107.95) (end 234.95 124.44476) (width 0.25) (layer F.Cu) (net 2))
 (segment (start 232.71226 109.52226) (end 232.71226 124.74702) (width 0.25) (layer B.Cu) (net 3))
 (segment (start 228.6 105.41) (end 232.71226 109.52226) (width 0.25) (layer B.Cu) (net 3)))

